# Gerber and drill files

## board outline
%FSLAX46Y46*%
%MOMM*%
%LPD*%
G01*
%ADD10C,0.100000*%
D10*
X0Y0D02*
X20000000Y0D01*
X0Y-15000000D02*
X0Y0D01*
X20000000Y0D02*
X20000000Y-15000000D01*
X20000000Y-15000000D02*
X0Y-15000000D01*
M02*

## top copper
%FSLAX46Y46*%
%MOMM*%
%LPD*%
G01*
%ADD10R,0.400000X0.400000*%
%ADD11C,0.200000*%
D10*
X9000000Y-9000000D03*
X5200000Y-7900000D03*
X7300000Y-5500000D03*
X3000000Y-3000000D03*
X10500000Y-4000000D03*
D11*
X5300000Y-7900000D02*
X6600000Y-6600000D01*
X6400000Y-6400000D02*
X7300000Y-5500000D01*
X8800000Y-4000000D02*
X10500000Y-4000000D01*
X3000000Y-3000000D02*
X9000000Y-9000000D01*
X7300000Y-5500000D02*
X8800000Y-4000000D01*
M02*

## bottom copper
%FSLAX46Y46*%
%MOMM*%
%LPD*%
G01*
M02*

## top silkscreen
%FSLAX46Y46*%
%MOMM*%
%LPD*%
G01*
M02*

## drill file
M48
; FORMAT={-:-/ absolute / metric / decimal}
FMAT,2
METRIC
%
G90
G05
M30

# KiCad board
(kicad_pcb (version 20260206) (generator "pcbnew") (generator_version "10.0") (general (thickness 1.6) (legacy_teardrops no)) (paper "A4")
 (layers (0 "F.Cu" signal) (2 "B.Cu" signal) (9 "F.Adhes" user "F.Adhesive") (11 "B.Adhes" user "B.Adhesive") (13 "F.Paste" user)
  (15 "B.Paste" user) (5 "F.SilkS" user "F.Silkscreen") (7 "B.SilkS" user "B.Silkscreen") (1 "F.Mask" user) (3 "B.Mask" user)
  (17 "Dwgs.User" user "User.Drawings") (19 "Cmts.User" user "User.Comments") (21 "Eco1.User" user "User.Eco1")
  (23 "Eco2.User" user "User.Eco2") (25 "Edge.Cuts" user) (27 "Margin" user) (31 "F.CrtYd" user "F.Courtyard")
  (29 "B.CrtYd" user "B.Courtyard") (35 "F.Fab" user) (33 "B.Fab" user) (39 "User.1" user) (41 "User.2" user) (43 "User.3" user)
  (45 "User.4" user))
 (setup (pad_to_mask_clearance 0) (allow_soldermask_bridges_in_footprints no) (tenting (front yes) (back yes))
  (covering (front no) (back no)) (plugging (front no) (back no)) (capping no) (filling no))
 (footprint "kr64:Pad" (layer "F.Cu") (at 9 9)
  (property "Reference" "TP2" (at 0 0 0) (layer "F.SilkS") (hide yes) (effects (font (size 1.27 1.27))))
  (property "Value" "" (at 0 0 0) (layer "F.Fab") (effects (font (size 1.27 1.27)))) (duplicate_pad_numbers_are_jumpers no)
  (pad "1" smd rect (at 0 0) (size 0.4 0.4) (layers "F.Cu" "F.Mask" "F.Paste") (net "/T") (thermal_bridge_angle 45)))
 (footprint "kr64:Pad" (layer "F.Cu") (at 5.2 7.9)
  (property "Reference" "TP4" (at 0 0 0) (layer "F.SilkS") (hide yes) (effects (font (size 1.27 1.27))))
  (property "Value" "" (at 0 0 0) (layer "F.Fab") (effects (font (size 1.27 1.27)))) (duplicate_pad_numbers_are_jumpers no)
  (pad "1" smd rect (at 0 0) (size 0.4 0.4) (layers "F.Cu" "F.Mask" "F.Paste") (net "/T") (thermal_bridge_angle 45)))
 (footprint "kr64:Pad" (layer "F.Cu") (at 7.3 5.5)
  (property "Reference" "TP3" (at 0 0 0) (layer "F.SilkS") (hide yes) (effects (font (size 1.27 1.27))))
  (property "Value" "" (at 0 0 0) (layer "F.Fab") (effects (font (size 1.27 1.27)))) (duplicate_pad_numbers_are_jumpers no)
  (pad "1" smd rect (at 0 0) (size 0.4 0.4) (layers "F.Cu" "F.Mask" "F.Paste") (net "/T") (thermal_bridge_angle 45)))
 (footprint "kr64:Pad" (layer "F.Cu") (at 3 3)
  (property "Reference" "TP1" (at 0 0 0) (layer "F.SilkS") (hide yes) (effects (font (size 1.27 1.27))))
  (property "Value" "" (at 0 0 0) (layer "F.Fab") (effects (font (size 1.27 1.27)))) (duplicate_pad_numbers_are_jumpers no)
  (pad "1" smd rect (at 0 0) (size 0.4 0.4) (layers "F.Cu" "F.Mask" "F.Paste") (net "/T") (thermal_bridge_angle 45)))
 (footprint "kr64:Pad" (layer "F.Cu") (at 10.5 4)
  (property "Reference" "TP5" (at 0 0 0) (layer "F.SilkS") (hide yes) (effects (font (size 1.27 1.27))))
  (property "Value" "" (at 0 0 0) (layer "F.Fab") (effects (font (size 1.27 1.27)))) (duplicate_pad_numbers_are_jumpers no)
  (pad "1" smd rect (at 0 0) (size 0.4 0.4) (layers "F.Cu" "F.Mask" "F.Paste") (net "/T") (thermal_bridge_angle 45)))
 (gr_line (start 0 0) (end 20 0) (stroke (width 0.1) (type default)) (layer "Edge.Cuts"))
 (gr_line (start 0 15) (end 0 0) (stroke (width 0.1) (type default)) (layer "Edge.Cuts"))
 (gr_line (start 20 0) (end 20 15) (stroke (width 0.1) (type default)) (layer "Edge.Cuts"))
 (gr_line (start 20 15) (end 0 15) (stroke (width 0.1) (type default)) (layer "Edge.Cuts"))
 (segment (start 5.3 7.9) (end 6.6 6.6) (width 0.2) (layer "F.Cu") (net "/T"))
 (segment (start 6.4 6.4) (end 7.3 5.5) (width 0.2) (layer "F.Cu") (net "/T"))
 (segment (start 8.8 4) (end 10.5 4) (width 0.2) (layer "F.Cu") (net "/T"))
 (segment (start 3 3) (end 9 9) (width 0.2) (layer "F.Cu") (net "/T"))
 (segment (start 7.3 5.5) (end 8.8 4) (width 0.2) (layer "F.Cu") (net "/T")))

